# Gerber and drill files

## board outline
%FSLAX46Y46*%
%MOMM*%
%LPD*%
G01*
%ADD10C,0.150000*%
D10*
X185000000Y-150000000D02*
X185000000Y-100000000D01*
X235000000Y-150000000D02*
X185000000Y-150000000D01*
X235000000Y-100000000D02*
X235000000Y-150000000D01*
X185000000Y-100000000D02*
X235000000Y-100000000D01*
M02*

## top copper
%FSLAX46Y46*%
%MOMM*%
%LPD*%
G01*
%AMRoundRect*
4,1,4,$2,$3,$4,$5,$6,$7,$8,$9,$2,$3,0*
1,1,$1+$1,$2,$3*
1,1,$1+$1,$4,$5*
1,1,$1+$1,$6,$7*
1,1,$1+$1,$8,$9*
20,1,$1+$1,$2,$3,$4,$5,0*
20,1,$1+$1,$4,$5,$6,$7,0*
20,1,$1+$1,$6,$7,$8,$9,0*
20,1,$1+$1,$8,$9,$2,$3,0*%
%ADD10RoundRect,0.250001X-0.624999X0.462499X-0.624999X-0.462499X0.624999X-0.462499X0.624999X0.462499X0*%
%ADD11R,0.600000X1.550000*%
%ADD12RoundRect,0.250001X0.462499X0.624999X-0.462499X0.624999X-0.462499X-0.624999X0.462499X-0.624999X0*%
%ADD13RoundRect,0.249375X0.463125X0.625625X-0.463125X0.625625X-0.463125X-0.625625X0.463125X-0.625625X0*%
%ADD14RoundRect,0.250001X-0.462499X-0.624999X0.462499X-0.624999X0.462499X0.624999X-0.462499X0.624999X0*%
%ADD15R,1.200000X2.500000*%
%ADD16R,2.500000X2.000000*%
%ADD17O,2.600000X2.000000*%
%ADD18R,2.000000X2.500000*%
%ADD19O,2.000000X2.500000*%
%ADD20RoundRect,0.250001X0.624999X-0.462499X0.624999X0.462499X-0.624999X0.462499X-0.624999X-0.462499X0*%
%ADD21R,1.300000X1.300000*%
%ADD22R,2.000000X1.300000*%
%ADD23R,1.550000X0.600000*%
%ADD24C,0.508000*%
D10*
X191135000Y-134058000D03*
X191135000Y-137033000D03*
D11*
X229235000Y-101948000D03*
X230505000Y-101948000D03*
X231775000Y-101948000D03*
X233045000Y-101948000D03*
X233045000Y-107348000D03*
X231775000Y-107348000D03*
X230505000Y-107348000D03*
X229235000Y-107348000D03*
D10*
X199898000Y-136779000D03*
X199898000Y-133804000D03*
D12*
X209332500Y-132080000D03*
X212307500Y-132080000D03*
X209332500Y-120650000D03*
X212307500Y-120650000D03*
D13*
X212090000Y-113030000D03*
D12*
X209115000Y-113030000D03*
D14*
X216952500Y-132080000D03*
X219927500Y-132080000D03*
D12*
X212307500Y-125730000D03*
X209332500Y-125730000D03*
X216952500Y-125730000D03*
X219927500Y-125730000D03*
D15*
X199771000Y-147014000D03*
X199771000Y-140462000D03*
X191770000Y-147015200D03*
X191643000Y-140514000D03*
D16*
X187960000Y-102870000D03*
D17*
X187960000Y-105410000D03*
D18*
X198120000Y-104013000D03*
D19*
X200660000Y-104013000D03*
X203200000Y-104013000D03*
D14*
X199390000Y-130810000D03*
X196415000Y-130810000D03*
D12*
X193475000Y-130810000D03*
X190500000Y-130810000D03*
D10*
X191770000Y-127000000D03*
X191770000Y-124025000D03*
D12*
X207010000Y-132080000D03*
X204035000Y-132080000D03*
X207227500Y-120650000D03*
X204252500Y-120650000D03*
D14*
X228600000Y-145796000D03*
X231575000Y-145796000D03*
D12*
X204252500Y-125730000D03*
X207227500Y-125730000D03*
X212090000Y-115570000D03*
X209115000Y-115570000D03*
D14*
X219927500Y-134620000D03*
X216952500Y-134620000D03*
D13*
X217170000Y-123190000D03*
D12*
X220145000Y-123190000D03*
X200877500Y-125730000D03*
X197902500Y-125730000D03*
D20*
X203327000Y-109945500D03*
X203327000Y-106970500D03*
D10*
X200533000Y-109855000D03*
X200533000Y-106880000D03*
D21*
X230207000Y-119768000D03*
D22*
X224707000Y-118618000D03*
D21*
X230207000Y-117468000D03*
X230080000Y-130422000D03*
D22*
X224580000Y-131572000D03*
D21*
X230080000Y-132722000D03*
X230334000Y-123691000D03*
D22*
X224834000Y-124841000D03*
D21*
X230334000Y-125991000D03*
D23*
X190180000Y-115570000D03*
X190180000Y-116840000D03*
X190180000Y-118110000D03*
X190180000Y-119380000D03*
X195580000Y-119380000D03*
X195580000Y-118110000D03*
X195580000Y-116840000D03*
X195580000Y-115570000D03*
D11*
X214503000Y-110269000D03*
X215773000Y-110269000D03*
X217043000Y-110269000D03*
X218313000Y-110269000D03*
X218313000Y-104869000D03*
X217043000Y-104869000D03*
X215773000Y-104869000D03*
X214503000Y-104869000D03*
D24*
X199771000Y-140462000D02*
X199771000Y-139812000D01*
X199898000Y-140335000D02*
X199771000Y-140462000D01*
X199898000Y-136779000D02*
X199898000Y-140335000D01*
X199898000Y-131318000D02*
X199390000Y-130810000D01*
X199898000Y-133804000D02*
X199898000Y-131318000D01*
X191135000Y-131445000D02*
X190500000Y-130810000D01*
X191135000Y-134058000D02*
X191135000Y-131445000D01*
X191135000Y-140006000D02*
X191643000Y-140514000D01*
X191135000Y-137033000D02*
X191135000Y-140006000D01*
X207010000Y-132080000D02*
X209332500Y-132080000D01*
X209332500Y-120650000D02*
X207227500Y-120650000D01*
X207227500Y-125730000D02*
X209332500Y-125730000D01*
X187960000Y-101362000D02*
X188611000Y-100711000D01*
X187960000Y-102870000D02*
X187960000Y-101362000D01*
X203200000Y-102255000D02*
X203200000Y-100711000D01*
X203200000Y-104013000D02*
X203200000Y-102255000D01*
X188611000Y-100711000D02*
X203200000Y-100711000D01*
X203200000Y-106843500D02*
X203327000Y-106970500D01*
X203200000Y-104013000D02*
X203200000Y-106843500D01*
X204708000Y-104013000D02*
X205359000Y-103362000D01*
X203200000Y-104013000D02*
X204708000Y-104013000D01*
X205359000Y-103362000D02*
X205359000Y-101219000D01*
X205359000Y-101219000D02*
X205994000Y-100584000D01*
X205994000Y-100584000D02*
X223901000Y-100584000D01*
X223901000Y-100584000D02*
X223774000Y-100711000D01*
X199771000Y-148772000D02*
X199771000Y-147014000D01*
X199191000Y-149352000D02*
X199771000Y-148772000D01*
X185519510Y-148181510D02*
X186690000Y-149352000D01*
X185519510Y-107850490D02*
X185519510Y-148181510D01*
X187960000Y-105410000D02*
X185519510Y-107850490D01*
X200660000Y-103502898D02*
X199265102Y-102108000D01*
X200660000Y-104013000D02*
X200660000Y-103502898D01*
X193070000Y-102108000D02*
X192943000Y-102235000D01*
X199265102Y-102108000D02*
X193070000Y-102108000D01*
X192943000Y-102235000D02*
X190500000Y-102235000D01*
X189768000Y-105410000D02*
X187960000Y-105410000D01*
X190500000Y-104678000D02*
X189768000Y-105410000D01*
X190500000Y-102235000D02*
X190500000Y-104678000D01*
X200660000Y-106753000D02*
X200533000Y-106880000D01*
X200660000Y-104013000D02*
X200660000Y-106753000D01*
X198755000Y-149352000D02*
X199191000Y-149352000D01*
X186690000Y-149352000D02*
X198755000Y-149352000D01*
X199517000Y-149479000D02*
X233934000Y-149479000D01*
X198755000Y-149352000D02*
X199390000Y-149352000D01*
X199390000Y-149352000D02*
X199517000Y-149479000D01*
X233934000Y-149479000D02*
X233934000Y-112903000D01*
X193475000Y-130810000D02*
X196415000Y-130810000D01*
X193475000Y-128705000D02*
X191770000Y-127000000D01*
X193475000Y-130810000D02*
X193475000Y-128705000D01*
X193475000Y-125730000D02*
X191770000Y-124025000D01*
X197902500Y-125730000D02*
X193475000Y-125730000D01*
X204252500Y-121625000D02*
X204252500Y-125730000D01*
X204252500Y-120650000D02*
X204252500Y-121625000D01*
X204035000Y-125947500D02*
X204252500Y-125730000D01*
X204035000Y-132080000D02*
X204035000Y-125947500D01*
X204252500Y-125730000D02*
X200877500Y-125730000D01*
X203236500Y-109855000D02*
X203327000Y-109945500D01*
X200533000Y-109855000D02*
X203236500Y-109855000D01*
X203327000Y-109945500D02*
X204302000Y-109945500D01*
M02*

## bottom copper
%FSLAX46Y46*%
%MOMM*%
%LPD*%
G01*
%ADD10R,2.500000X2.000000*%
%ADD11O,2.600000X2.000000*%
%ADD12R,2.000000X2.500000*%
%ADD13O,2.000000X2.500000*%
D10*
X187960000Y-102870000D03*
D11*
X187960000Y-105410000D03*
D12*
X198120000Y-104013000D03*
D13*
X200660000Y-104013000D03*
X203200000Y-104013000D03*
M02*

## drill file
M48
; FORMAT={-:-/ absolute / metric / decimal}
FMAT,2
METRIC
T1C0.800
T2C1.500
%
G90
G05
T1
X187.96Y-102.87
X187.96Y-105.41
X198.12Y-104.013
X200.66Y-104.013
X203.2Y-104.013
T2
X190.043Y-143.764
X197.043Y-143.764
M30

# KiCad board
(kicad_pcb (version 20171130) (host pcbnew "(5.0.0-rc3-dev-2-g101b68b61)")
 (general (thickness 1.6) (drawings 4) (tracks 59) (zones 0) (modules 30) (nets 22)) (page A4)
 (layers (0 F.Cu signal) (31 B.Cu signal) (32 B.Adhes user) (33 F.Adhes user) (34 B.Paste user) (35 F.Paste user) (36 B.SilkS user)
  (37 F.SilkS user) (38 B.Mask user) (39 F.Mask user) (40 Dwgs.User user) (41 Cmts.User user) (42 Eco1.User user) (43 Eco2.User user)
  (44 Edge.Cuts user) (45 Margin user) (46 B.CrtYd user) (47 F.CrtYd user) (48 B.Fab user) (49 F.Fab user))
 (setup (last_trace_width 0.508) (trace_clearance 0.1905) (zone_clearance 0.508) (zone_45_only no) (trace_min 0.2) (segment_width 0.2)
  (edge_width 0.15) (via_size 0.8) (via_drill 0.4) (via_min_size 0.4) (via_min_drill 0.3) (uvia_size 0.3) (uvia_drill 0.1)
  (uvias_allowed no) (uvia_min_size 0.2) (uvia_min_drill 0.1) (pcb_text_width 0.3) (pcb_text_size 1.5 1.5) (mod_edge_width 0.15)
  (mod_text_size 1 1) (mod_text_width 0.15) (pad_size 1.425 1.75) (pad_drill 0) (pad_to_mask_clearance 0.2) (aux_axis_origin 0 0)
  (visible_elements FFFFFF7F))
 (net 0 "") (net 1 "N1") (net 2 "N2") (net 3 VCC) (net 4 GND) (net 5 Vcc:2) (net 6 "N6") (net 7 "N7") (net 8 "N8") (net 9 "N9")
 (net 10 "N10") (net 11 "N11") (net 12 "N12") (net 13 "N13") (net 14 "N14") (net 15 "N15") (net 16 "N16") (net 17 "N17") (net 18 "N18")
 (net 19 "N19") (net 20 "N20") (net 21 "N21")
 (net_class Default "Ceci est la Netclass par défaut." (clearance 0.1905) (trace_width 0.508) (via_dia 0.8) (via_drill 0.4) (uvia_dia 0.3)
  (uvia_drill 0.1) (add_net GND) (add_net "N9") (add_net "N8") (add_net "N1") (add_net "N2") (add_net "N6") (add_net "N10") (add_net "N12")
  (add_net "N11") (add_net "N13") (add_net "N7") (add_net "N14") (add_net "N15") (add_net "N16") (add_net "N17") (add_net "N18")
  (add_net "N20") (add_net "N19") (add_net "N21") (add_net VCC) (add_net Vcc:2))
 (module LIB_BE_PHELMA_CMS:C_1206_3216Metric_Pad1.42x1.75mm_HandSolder (layer F.Cu) (at 191.135 135.5455 270)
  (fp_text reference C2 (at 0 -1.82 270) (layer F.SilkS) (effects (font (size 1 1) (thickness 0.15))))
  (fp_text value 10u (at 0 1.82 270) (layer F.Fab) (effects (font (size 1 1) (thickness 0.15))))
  (pad 1 smd roundrect (at -1.4875 0 270) (size 1.425 1.75) (layers F.Cu F.Paste F.Mask) (roundrect_rratio 0.175439) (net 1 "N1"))
  (pad 2 smd roundrect (at 1.4875 0 270) (size 1.425 1.75) (layers F.Cu F.Paste F.Mask) (roundrect_rratio 0.175439) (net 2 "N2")))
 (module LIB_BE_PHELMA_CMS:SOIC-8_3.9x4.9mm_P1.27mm (layer F.Cu) (at 231.14 104.648 90)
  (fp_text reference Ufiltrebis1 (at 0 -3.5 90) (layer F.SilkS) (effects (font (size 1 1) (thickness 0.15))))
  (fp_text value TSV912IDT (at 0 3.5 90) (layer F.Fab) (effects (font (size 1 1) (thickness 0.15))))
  (pad 8 smd rect (at 2.7 -1.905 90) (size 1.55 0.6) (layers F.Cu F.Paste F.Mask) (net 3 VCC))
  (pad 7 smd rect (at 2.7 -0.635 90) (size 1.55 0.6) (layers F.Cu F.Paste F.Mask))
  (pad 6 smd rect (at 2.7 0.635 90) (size 1.55 0.6) (layers F.Cu F.Paste F.Mask))
  (pad 5 smd rect (at 2.7 1.905 90) (size 1.55 0.6) (layers F.Cu F.Paste F.Mask))
  (pad 4 smd rect (at -2.7 1.905 90) (size 1.55 0.6) (layers F.Cu F.Paste F.Mask) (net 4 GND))
  (pad 3 smd rect (at -2.7 0.635 90) (size 1.55 0.6) (layers F.Cu F.Paste F.Mask) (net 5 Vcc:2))
  (pad 2 smd rect (at -2.7 -0.635 90) (size 1.55 0.6) (layers F.Cu F.Paste F.Mask) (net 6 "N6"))
  (pad 1 smd rect (at -2.7 -1.905 90) (size 1.55 0.6) (layers F.Cu F.Paste F.Mask) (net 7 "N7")))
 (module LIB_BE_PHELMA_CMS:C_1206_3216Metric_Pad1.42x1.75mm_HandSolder (layer F.Cu) (at 199.898 135.2915 270)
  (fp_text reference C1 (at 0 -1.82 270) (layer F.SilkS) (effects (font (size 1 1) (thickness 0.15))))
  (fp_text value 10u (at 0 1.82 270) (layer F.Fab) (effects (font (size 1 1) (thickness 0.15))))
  (pad 2 smd roundrect (at 1.4875 0 270) (size 1.425 1.75) (layers F.Cu F.Paste F.Mask) (roundrect_rratio 0.175439) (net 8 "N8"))
  (pad 1 smd roundrect (at -1.4875 0 270) (size 1.425 1.75) (layers F.Cu F.Paste F.Mask) (roundrect_rratio 0.175439) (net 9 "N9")))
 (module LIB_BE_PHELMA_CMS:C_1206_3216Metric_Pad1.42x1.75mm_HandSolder (layer F.Cu) (at 210.82 132.08 180)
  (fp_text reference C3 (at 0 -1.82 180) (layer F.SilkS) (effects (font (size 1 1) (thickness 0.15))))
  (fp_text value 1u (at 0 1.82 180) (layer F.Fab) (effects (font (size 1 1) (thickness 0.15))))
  (pad 2 smd roundrect (at 1.4875 0 180) (size 1.425 1.75) (layers F.Cu F.Paste F.Mask) (roundrect_rratio 0.175439) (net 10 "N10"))
  (pad 1 smd roundrect (at -1.4875 0 180) (size 1.425 1.75) (layers F.Cu F.Paste F.Mask) (roundrect_rratio 0.175439) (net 6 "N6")))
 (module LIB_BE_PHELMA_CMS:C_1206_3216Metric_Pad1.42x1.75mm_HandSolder (layer F.Cu) (at 210.82 120.65 180)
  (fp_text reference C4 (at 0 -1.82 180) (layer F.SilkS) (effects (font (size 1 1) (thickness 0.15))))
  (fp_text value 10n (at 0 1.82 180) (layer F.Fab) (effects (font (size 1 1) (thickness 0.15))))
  (pad 2 smd roundrect (at 1.4875 0 180) (size 1.425 1.75) (layers F.Cu F.Paste F.Mask) (roundrect_rratio 0.175439) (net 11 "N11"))
  (pad 1 smd roundrect (at -1.4875 0 180) (size 1.425 1.75) (layers F.Cu F.Paste F.Mask) (roundrect_rratio 0.175439) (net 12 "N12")))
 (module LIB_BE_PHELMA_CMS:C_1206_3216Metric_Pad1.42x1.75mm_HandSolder (layer F.Cu) (at 210.6025 113.03 180)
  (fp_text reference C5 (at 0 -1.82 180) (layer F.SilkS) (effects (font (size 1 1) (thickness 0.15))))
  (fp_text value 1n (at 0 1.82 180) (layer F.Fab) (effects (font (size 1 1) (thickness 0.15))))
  (pad 1 smd roundrect (at -1.4875 0 180) (size 1.425 1.75) (layers F.Cu F.Paste F.Mask) (roundrect_rratio 0.175) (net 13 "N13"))
  (pad 2 smd roundrect (at 1.4875 0 180) (size 1.425 1.75) (layers F.Cu F.Paste F.Mask) (roundrect_rratio 0.175439) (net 12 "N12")))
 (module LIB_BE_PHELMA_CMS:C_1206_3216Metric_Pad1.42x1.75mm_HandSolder (layer F.Cu) (at 218.44 132.08)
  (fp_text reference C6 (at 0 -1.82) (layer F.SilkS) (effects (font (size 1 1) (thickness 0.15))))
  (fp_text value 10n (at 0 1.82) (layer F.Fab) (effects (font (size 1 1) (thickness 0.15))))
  (pad 1 smd roundrect (at -1.4875 0) (size 1.425 1.75) (layers F.Cu F.Paste F.Mask) (roundrect_rratio 0.175439) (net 7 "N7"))
  (pad 2 smd roundrect (at 1.4875 0) (size 1.425 1.75) (layers F.Cu F.Paste F.Mask) (roundrect_rratio 0.175439) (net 6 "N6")))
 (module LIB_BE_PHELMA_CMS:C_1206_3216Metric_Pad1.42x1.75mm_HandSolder (layer F.Cu) (at 210.82 125.73 180)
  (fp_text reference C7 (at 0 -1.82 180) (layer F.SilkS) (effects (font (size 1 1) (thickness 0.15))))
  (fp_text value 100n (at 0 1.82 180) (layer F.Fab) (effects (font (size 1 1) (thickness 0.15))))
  (pad 1 smd roundrect (at -1.4875 0 180) (size 1.425 1.75) (layers F.Cu F.Paste F.Mask) (roundrect_rratio 0.175439) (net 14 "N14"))
  (pad 2 smd roundrect (at 1.4875 0 180) (size 1.425 1.75) (layers F.Cu F.Paste F.Mask) (roundrect_rratio 0.175439) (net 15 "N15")))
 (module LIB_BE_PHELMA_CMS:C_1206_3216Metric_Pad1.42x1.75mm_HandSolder (layer F.Cu) (at 218.44 125.73 180)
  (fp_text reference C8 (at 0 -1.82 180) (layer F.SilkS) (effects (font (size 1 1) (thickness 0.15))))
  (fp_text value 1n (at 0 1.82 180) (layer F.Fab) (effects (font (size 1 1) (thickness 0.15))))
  (pad 2 smd roundrect (at 1.4875 0 180) (size 1.425 1.75) (layers F.Cu F.Paste F.Mask) (roundrect_rratio 0.175439) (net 14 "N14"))
  (pad 1 smd roundrect (at -1.4875 0 180) (size 1.425 1.75) (layers F.Cu F.Paste F.Mask) (roundrect_rratio 0.175439) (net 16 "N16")))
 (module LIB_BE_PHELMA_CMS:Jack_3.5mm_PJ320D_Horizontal (layer F.Cu) (at 194.818 143.764)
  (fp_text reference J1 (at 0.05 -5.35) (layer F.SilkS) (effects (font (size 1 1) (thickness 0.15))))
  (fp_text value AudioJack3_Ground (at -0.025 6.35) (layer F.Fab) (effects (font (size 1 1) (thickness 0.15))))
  (pad S smd rect (at 4.953 3.25) (size 1.2 2.5) (layers F.Cu F.Paste F.Mask) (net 4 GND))
  (pad R smd rect (at 4.953 -3.302) (size 1.2 2.5) (layers F.Cu F.Paste F.Mask) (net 8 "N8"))
  (pad T smd rect (at -3.048 3.2512) (size 1.2 2.5) (layers F.Cu F.Paste F.Mask) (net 2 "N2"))
  (pad T smd rect (at -3.175 -3.25) (size 1.2 2.5) (layers F.Cu F.Paste F.Mask) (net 2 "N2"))
  (pad "" np_thru_hole circle (at -4.775 0) (size 1.5 1.5) (drill 1.5) (layers *.Cu *.Mask))
  (pad "" np_thru_hole circle (at 2.225 0) (size 1.5 1.5) (drill 1.5) (layers *.Cu *.Mask)))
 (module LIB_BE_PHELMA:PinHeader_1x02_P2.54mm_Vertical (layer F.Cu) (at 187.96 102.87)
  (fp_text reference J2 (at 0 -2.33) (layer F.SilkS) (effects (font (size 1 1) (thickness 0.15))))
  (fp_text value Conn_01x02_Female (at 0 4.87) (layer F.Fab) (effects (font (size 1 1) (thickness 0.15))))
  (pad 1 thru_hole rect (at 0 0) (size 2.5 2) (drill 0.8) (layers *.Cu *.Mask) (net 3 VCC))
  (pad 2 thru_hole oval (at 0 2.54) (size 2.6 2) (drill 0.8) (layers *.Cu *.Mask) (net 4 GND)))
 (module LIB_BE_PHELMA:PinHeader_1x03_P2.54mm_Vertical (layer F.Cu) (at 198.12 104.013 90)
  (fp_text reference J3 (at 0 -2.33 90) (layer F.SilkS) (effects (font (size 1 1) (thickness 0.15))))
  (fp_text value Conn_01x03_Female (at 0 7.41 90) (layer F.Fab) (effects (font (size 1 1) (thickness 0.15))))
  (pad 1 thru_hole rect (at 0 0 90) (size 2.5 2) (drill 0.8) (layers *.Cu *.Mask) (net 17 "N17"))
  (pad 2 thru_hole oval (at 0 2.54 90) (size 2.5 2) (drill 0.8) (layers *.Cu *.Mask) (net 4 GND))
  (pad 3 thru_hole oval (at 0 5.08 90) (size 2.5 2) (drill 0.8) (layers *.Cu *.Mask) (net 3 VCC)))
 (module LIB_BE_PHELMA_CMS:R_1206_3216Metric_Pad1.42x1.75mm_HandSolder (layer F.Cu) (at 197.9025 130.81)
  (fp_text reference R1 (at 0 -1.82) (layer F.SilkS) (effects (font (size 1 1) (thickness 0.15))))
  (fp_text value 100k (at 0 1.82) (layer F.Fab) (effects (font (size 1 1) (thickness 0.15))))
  (pad 2 smd roundrect (at 1.4875 0) (size 1.425 1.75) (layers F.Cu F.Paste F.Mask) (roundrect_rratio 0.175439) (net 9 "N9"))
  (pad 1 smd roundrect (at -1.4875 0) (size 1.425 1.75) (layers F.Cu F.Paste F.Mask) (roundrect_rratio 0.175439) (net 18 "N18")))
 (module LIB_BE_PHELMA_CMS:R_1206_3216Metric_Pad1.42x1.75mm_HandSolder (layer F.Cu) (at 191.9875 130.81 180)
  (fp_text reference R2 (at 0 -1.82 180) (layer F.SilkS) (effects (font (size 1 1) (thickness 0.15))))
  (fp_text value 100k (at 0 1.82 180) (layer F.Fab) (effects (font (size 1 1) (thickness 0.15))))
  (pad 1 smd roundrect (at -1.4875 0 180) (size 1.425 1.75) (layers F.Cu F.Paste F.Mask) (roundrect_rratio 0.175439) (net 18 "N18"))
  (pad 2 smd roundrect (at 1.4875 0 180) (size 1.425 1.75) (layers F.Cu F.Paste F.Mask) (roundrect_rratio 0.175439) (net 1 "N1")))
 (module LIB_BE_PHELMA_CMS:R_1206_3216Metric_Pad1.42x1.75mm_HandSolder (layer F.Cu) (at 191.77 125.5125 270)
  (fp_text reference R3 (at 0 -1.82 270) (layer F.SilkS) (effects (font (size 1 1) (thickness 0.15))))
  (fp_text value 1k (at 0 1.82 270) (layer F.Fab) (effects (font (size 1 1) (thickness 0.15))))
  (pad 2 smd roundrect (at 1.4875 0 270) (size 1.425 1.75) (layers F.Cu F.Paste F.Mask) (roundrect_rratio 0.175439) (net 18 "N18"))
  (pad 1 smd roundrect (at -1.4875 0 270) (size 1.425 1.75) (layers F.Cu F.Paste F.Mask) (roundrect_rratio 0.175439) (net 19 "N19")))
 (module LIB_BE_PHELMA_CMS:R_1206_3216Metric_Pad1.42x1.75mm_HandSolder (layer F.Cu) (at 205.5225 132.08 180)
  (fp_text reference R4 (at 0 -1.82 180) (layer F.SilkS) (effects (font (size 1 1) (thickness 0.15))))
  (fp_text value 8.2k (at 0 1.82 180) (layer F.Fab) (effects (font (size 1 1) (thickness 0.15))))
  (pad 1 smd roundrect (at -1.4875 0 180) (size 1.425 1.75) (layers F.Cu F.Paste F.Mask) (roundrect_rratio 0.175439) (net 10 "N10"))
  (pad 2 smd roundrect (at 1.4875 0 180) (size 1.425 1.75) (layers F.Cu F.Paste F.Mask) (roundrect_rratio 0.175439) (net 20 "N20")))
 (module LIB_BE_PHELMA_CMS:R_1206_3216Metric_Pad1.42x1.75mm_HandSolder (layer F.Cu) (at 205.74 120.65 180)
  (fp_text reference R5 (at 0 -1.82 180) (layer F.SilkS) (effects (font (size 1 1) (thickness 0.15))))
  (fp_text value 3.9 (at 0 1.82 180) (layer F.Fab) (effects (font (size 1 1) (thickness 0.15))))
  (pad 1 smd roundrect (at -1.4875 0 180) (size 1.425 1.75) (layers F.Cu F.Paste F.Mask) (roundrect_rratio 0.175439) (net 11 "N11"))
  (pad 2 smd roundrect (at 1.4875 0 180) (size 1.425 1.75) (layers F.Cu F.Paste F.Mask) (roundrect_rratio 0.175439) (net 20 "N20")))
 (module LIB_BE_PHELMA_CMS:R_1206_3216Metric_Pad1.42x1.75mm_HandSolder (layer F.Cu) (at 230.0875 145.796)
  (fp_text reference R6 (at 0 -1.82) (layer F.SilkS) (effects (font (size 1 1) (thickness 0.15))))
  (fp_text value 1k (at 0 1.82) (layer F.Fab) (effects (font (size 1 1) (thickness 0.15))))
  (pad 1 smd roundrect (at -1.4875 0) (size 1.425 1.75) (layers F.Cu F.Paste F.Mask) (roundrect_rratio 0.175439) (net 17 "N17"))
  (pad 2 smd roundrect (at 1.4875 0) (size 1.425 1.75) (layers F.Cu F.Paste F.Mask) (roundrect_rratio 0.175439) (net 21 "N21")))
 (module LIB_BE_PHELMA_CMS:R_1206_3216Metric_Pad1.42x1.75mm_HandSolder (layer F.Cu) (at 205.74 125.73 180)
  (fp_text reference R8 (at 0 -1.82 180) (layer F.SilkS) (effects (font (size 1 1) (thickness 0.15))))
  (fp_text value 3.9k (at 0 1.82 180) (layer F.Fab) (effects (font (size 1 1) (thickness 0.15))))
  (pad 2 smd roundrect (at 1.4875 0 180) (size 1.425 1.75) (layers F.Cu F.Paste F.Mask) (roundrect_rratio 0.175439) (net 20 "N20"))
  (pad 1 smd roundrect (at -1.4875 0 180) (size 1.425 1.75) (layers F.Cu F.Paste F.Mask) (roundrect_rratio 0.175439) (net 15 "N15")))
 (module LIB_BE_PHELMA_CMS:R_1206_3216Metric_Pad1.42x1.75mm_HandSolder (layer F.Cu) (at 210.6025 115.57 180)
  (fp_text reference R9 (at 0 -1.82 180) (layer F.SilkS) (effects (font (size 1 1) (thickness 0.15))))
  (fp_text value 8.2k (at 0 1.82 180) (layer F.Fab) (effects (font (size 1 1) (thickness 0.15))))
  (pad 1 smd roundrect (at -1.4875 0 180) (size 1.425 1.75) (layers F.Cu F.Paste F.Mask) (roundrect_rratio 0.175439) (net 13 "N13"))
  (pad 2 smd roundrect (at 1.4875 0 180) (size 1.425 1.75) (layers F.Cu F.Paste F.Mask) (roundrect_rratio 0.175439) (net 12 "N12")))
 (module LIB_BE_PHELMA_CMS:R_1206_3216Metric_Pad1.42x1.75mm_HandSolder (layer F.Cu) (at 218.44 134.62)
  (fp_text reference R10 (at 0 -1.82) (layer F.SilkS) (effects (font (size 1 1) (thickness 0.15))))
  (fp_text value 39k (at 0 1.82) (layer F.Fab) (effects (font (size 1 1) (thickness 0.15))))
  (pad 2 smd roundrect (at 1.4875 0) (size 1.425 1.75) (layers F.Cu F.Paste F.Mask) (roundrect_rratio 0.175439) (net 6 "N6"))
  (pad 1 smd roundrect (at -1.4875 0) (size 1.425 1.75) (layers F.Cu F.Paste F.Mask) (roundrect_rratio 0.175439) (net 7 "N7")))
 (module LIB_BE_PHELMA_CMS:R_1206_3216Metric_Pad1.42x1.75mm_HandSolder (layer F.Cu) (at 218.6575 123.19 180)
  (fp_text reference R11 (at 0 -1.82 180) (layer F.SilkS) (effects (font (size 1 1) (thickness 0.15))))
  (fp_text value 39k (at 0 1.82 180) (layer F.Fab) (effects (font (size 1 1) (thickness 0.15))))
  (pad 2 smd roundrect (at 1.4875 0 180) (size 1.425 1.75) (layers F.Cu F.Paste F.Mask) (roundrect_rratio 0.175) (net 14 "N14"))
  (pad 1 smd roundrect (at -1.4875 0 180) (size 1.425 1.75) (layers F.Cu F.Paste F.Mask) (roundrect_rratio 0.175439) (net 16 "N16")))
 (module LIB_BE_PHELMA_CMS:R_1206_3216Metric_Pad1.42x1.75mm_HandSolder (layer F.Cu) (at 199.39 125.73 180)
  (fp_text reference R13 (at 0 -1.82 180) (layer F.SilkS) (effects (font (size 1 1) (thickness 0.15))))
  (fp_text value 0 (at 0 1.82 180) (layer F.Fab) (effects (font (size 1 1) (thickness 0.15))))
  (pad 1 smd roundrect (at -1.4875 0 180) (size 1.425 1.75) (layers F.Cu F.Paste F.Mask) (roundrect_rratio 0.175439) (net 20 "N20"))
  (pad 2 smd roundrect (at 1.4875 0 180) (size 1.425 1.75) (layers F.Cu F.Paste F.Mask) (roundrect_rratio 0.175439) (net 19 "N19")))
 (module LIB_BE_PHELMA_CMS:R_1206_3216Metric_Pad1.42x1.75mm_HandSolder (layer F.Cu) (at 203.327 108.458 90)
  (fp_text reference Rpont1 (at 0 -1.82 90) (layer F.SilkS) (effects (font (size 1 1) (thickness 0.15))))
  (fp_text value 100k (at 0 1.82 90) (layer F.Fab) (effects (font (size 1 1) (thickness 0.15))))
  (pad 1 smd roundrect (at -1.4875 0 90) (size 1.425 1.75) (layers F.Cu F.Paste F.Mask) (roundrect_rratio 0.175439) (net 5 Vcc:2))
  (pad 2 smd roundrect (at 1.4875 0 90) (size 1.425 1.75) (layers F.Cu F.Paste F.Mask) (roundrect_rratio 0.175439) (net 3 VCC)))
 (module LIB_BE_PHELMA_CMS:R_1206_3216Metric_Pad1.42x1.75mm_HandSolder (layer F.Cu) (at 200.533 108.3675 270)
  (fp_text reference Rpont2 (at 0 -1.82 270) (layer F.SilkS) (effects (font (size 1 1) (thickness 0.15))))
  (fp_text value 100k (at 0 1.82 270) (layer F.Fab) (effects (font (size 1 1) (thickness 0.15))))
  (pad 2 smd roundrect (at 1.4875 0 270) (size 1.425 1.75) (layers F.Cu F.Paste F.Mask) (roundrect_rratio 0.175439) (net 5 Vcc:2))
  (pad 1 smd roundrect (at -1.4875 0 270) (size 1.425 1.75) (layers F.Cu F.Paste F.Mask) (roundrect_rratio 0.175439) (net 4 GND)))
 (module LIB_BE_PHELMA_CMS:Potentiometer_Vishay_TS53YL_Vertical (layer F.Cu) (at 227.457 118.618)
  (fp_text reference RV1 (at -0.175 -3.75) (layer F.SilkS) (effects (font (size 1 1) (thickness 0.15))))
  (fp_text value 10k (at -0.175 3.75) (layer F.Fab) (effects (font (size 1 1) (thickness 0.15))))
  (pad 3 smd rect (at 2.75 1.15) (size 1.3 1.3) (layers F.Cu F.Paste F.Mask) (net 21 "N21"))
  (pad 2 smd rect (at -2.75 0) (size 2 1.3) (layers F.Cu F.Paste F.Mask) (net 13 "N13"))
  (pad 1 smd rect (at 2.75 -1.15) (size 1.3 1.3) (layers F.Cu F.Paste F.Mask) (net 13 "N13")))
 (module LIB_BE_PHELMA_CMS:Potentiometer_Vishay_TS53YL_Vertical (layer F.Cu) (at 227.33 131.572)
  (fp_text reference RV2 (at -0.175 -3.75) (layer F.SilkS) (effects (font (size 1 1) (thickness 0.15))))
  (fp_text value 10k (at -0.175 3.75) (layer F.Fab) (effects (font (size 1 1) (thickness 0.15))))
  (pad 1 smd rect (at 2.75 -1.15) (size 1.3 1.3) (layers F.Cu F.Paste F.Mask) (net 21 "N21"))
  (pad 2 smd rect (at -2.75 0) (size 2 1.3) (layers F.Cu F.Paste F.Mask) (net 7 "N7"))
  (pad 3 smd rect (at 2.75 1.15) (size 1.3 1.3) (layers F.Cu F.Paste F.Mask) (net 7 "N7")))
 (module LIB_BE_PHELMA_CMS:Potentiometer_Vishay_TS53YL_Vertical (layer F.Cu) (at 227.584 124.841)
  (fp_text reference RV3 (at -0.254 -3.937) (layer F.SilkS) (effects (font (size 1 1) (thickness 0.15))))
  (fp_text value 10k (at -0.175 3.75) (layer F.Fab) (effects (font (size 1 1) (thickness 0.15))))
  (pad 1 smd rect (at 2.75 -1.15) (size 1.3 1.3) (layers F.Cu F.Paste F.Mask) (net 16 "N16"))
  (pad 2 smd rect (at -2.75 0) (size 2 1.3) (layers F.Cu F.Paste F.Mask) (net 16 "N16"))
  (pad 3 smd rect (at 2.75 1.15) (size 1.3 1.3) (layers F.Cu F.Paste F.Mask) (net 21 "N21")))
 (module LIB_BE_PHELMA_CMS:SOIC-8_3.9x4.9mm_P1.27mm (layer F.Cu) (at 192.88 117.475)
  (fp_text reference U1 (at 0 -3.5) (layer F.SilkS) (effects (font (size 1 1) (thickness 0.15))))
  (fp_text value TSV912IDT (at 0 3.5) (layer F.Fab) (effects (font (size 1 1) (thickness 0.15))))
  (pad 1 smd rect (at -2.7 -1.905) (size 1.55 0.6) (layers F.Cu F.Paste F.Mask) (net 19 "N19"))
  (pad 2 smd rect (at -2.7 -0.635) (size 1.55 0.6) (layers F.Cu F.Paste F.Mask) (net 18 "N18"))
  (pad 3 smd rect (at -2.7 0.635) (size 1.55 0.6) (layers F.Cu F.Paste F.Mask) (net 5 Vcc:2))
  (pad 4 smd rect (at -2.7 1.905) (size 1.55 0.6) (layers F.Cu F.Paste F.Mask) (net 4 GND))
  (pad 5 smd rect (at 2.7 1.905) (size 1.55 0.6) (layers F.Cu F.Paste F.Mask) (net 5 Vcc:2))
  (pad 6 smd rect (at 2.7 0.635) (size 1.55 0.6) (layers F.Cu F.Paste F.Mask) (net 21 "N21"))
  (pad 7 smd rect (at 2.7 -0.635) (size 1.55 0.6) (layers F.Cu F.Paste F.Mask) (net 17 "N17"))
  (pad 8 smd rect (at 2.7 -1.905) (size 1.55 0.6) (layers F.Cu F.Paste F.Mask) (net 3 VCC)))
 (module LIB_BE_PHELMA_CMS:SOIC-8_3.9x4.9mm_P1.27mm (layer F.Cu) (at 216.408 107.569 90)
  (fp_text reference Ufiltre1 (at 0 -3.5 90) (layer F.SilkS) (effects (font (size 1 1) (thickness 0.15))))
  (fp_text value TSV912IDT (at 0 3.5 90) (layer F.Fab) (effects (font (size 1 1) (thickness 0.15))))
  (pad 1 smd rect (at -2.7 -1.905 90) (size 1.55 0.6) (layers F.Cu F.Paste F.Mask) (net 13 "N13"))
  (pad 2 smd rect (at -2.7 -0.635 90) (size 1.55 0.6) (layers F.Cu F.Paste F.Mask) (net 12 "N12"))
  (pad 3 smd rect (at -2.7 0.635 90) (size 1.55 0.6) (layers F.Cu F.Paste F.Mask) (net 5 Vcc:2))
  (pad 4 smd rect (at -2.7 1.905 90) (size 1.55 0.6) (layers F.Cu F.Paste F.Mask) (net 4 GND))
  (pad 5 smd rect (at 2.7 1.905 90) (size 1.55 0.6) (layers F.Cu F.Paste F.Mask) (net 5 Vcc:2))
  (pad 6 smd rect (at 2.7 0.635 90) (size 1.55 0.6) (layers F.Cu F.Paste F.Mask) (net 14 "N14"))
  (pad 7 smd rect (at 2.7 -0.635 90) (size 1.55 0.6) (layers F.Cu F.Paste F.Mask) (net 16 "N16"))
  (pad 8 smd rect (at 2.7 -1.905 90) (size 1.55 0.6) (layers F.Cu F.Paste F.Mask) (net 3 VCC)))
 (gr_line (start 185 150) (end 185 100) (layer Edge.Cuts) (width 0.15))
 (gr_line (start 235 150) (end 185 150) (layer Edge.Cuts) (width 0.15))
 (gr_line (start 235 100) (end 235 150) (layer Edge.Cuts) (width 0.15))
 (gr_line (start 185 100) (end 235 100) (layer Edge.Cuts) (width 0.15))
 (segment (start 199.771 140.462) (end 199.771 139.812) (width 0.508) (layer F.Cu) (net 8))
 (segment (start 199.898 140.335) (end 199.771 140.462) (width 0.508) (layer F.Cu) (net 8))
 (segment (start 199.898 136.779) (end 199.898 140.335) (width 0.508) (layer F.Cu) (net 8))
 (segment (start 199.898 131.318) (end 199.39 130.81) (width 0.508) (layer F.Cu) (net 9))
 (segment (start 199.898 133.804) (end 199.898 131.318) (width 0.508) (layer F.Cu) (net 9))
 (segment (start 191.135 131.445) (end 190.5 130.81) (width 0.508) (layer F.Cu) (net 1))
 (segment (start 191.135 134.058) (end 191.135 131.445) (width 0.508) (layer F.Cu) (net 1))
 (segment (start 191.135 140.006) (end 191.643 140.514) (width 0.508) (layer F.Cu) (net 2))
 (segment (start 191.135 137.033) (end 191.135 140.006) (width 0.508) (layer F.Cu) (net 2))
 (segment (start 207.01 132.08) (end 209.3325 132.08) (width 0.508) (layer F.Cu) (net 10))
 (segment (start 209.3325 120.65) (end 207.2275 120.65) (width 0.508) (layer F.Cu) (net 11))
 (segment (start 207.2275 125.73) (end 209.3325 125.73) (width 0.508) (layer F.Cu) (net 15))
 (segment (start 187.96 101.362) (end 188.611 100.711) (width 0.508) (layer F.Cu) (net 3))
 (segment (start 187.96 102.87) (end 187.96 101.362) (width 0.508) (layer F.Cu) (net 3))
 (segment (start 203.2 102.255) (end 203.2 100.711) (width 0.508) (layer F.Cu) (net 3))
 (segment (start 203.2 104.013) (end 203.2 102.255) (width 0.508) (layer F.Cu) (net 3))
 (segment (start 188.611 100.711) (end 203.2 100.711) (width 0.508) (layer F.Cu) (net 3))
 (segment (start 203.2 106.8435) (end 203.327 106.9705) (width 0.508) (layer F.Cu) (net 3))
 (segment (start 203.2 104.013) (end 203.2 106.8435) (width 0.508) (layer F.Cu) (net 3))
 (segment (start 204.708 104.013) (end 205.359 103.362) (width 0.508) (layer F.Cu) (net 3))
 (segment (start 203.2 104.013) (end 204.708 104.013) (width 0.508) (layer F.Cu) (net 3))
 (segment (start 205.359 103.362) (end 205.359 101.219) (width 0.508) (layer F.Cu) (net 3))
 (segment (start 205.359 101.219) (end 205.994 100.584) (width 0.508) (layer F.Cu) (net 3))
 (segment (start 205.994 100.584) (end 223.901 100.584) (width 0.508) (layer F.Cu) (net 3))
 (segment (start 223.901 100.584) (end 223.774 100.711) (width 0.508) (layer F.Cu) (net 3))
 (segment (start 199.771 148.772) (end 199.771 147.014) (width 0.508) (layer F.Cu) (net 4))
 (segment (start 199.191 149.352) (end 199.771 148.772) (width 0.508) (layer F.Cu) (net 4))
 (segment (start 185.51951 148.18151) (end 186.69 149.352) (width 0.508) (layer F.Cu) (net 4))
 (segment (start 185.51951 107.85049) (end 185.51951 148.18151) (width 0.508) (layer F.Cu) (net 4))
 (segment (start 187.96 105.41) (end 185.51951 107.85049) (width 0.508) (layer F.Cu) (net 4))
 (segment (start 200.66 103.502898) (end 199.265102 102.108) (width 0.508) (layer F.Cu) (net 4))
 (segment (start 200.66 104.013) (end 200.66 103.502898) (width 0.508) (layer F.Cu) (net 4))
 (segment (start 193.07 102.108) (end 192.943 102.235) (width 0.508) (layer F.Cu) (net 4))
 (segment (start 199.265102 102.108) (end 193.07 102.108) (width 0.508) (layer F.Cu) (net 4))
 (segment (start 192.943 102.235) (end 190.5 102.235) (width 0.508) (layer F.Cu) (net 4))
 (segment (start 189.768 105.41) (end 187.96 105.41) (width 0.508) (layer F.Cu) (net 4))
 (segment (start 190.5 104.678) (end 189.768 105.41) (width 0.508) (layer F.Cu) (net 4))
 (segment (start 190.5 102.235) (end 190.5 104.678) (width 0.508) (layer F.Cu) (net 4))
 (segment (start 200.66 106.753) (end 200.533 106.88) (width 0.508) (layer F.Cu) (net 4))
 (segment (start 200.66 104.013) (end 200.66 106.753) (width 0.508) (layer F.Cu) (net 4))
 (segment (start 198.755 149.352) (end 199.191 149.352) (width 0.508) (layer F.Cu) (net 4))
 (segment (start 186.69 149.352) (end 198.755 149.352) (width 0.508) (layer F.Cu) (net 4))
 (segment (start 199.517 149.479) (end 233.934 149.479) (width 0.508) (layer F.Cu) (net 4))
 (segment (start 198.755 149.352) (end 199.39 149.352) (width 0.508) (layer F.Cu) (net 4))
 (segment (start 199.39 149.352) (end 199.517 149.479) (width 0.508) (layer F.Cu) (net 4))
 (segment (start 233.934 149.479) (end 233.934 112.903) (width 0.508) (layer F.Cu) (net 4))
 (segment (start 193.475 130.81) (end 196.415 130.81) (width 0.508) (layer F.Cu) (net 18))
 (segment (start 193.475 128.705) (end 191.77 127) (width 0.508) (layer F.Cu) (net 18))
 (segment (start 193.475 130.81) (end 193.475 128.705) (width 0.508) (layer F.Cu) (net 18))
 (segment (start 193.475 125.73) (end 191.77 124.025) (width 0.508) (layer F.Cu) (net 19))
 (segment (start 197.9025 125.73) (end 193.475 125.73) (width 0.508) (layer F.Cu) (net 19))
 (segment (start 204.2525 121.625) (end 204.2525 125.73) (width 0.508) (layer F.Cu) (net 20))
 (segment (start 204.2525 120.65) (end 204.2525 121.625) (width 0.508) (layer F.Cu) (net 20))
 (segment (start 204.035 125.9475) (end 204.2525 125.73) (width 0.508) (layer F.Cu) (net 20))
 (segment (start 204.035 132.08) (end 204.035 125.9475) (width 0.508) (layer F.Cu) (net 20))
 (segment (start 204.2525 125.73) (end 200.8775 125.73) (width 0.508) (layer F.Cu) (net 20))
 (segment (start 203.2365 109.855) (end 203.327 109.9455) (width 0.508) (layer F.Cu) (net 5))
 (segment (start 200.533 109.855) (end 203.2365 109.855) (width 0.508) (layer F.Cu) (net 5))
 (segment (start 203.327 109.9455) (end 204.302 109.9455) (width 0.508) (layer F.Cu) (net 5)))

